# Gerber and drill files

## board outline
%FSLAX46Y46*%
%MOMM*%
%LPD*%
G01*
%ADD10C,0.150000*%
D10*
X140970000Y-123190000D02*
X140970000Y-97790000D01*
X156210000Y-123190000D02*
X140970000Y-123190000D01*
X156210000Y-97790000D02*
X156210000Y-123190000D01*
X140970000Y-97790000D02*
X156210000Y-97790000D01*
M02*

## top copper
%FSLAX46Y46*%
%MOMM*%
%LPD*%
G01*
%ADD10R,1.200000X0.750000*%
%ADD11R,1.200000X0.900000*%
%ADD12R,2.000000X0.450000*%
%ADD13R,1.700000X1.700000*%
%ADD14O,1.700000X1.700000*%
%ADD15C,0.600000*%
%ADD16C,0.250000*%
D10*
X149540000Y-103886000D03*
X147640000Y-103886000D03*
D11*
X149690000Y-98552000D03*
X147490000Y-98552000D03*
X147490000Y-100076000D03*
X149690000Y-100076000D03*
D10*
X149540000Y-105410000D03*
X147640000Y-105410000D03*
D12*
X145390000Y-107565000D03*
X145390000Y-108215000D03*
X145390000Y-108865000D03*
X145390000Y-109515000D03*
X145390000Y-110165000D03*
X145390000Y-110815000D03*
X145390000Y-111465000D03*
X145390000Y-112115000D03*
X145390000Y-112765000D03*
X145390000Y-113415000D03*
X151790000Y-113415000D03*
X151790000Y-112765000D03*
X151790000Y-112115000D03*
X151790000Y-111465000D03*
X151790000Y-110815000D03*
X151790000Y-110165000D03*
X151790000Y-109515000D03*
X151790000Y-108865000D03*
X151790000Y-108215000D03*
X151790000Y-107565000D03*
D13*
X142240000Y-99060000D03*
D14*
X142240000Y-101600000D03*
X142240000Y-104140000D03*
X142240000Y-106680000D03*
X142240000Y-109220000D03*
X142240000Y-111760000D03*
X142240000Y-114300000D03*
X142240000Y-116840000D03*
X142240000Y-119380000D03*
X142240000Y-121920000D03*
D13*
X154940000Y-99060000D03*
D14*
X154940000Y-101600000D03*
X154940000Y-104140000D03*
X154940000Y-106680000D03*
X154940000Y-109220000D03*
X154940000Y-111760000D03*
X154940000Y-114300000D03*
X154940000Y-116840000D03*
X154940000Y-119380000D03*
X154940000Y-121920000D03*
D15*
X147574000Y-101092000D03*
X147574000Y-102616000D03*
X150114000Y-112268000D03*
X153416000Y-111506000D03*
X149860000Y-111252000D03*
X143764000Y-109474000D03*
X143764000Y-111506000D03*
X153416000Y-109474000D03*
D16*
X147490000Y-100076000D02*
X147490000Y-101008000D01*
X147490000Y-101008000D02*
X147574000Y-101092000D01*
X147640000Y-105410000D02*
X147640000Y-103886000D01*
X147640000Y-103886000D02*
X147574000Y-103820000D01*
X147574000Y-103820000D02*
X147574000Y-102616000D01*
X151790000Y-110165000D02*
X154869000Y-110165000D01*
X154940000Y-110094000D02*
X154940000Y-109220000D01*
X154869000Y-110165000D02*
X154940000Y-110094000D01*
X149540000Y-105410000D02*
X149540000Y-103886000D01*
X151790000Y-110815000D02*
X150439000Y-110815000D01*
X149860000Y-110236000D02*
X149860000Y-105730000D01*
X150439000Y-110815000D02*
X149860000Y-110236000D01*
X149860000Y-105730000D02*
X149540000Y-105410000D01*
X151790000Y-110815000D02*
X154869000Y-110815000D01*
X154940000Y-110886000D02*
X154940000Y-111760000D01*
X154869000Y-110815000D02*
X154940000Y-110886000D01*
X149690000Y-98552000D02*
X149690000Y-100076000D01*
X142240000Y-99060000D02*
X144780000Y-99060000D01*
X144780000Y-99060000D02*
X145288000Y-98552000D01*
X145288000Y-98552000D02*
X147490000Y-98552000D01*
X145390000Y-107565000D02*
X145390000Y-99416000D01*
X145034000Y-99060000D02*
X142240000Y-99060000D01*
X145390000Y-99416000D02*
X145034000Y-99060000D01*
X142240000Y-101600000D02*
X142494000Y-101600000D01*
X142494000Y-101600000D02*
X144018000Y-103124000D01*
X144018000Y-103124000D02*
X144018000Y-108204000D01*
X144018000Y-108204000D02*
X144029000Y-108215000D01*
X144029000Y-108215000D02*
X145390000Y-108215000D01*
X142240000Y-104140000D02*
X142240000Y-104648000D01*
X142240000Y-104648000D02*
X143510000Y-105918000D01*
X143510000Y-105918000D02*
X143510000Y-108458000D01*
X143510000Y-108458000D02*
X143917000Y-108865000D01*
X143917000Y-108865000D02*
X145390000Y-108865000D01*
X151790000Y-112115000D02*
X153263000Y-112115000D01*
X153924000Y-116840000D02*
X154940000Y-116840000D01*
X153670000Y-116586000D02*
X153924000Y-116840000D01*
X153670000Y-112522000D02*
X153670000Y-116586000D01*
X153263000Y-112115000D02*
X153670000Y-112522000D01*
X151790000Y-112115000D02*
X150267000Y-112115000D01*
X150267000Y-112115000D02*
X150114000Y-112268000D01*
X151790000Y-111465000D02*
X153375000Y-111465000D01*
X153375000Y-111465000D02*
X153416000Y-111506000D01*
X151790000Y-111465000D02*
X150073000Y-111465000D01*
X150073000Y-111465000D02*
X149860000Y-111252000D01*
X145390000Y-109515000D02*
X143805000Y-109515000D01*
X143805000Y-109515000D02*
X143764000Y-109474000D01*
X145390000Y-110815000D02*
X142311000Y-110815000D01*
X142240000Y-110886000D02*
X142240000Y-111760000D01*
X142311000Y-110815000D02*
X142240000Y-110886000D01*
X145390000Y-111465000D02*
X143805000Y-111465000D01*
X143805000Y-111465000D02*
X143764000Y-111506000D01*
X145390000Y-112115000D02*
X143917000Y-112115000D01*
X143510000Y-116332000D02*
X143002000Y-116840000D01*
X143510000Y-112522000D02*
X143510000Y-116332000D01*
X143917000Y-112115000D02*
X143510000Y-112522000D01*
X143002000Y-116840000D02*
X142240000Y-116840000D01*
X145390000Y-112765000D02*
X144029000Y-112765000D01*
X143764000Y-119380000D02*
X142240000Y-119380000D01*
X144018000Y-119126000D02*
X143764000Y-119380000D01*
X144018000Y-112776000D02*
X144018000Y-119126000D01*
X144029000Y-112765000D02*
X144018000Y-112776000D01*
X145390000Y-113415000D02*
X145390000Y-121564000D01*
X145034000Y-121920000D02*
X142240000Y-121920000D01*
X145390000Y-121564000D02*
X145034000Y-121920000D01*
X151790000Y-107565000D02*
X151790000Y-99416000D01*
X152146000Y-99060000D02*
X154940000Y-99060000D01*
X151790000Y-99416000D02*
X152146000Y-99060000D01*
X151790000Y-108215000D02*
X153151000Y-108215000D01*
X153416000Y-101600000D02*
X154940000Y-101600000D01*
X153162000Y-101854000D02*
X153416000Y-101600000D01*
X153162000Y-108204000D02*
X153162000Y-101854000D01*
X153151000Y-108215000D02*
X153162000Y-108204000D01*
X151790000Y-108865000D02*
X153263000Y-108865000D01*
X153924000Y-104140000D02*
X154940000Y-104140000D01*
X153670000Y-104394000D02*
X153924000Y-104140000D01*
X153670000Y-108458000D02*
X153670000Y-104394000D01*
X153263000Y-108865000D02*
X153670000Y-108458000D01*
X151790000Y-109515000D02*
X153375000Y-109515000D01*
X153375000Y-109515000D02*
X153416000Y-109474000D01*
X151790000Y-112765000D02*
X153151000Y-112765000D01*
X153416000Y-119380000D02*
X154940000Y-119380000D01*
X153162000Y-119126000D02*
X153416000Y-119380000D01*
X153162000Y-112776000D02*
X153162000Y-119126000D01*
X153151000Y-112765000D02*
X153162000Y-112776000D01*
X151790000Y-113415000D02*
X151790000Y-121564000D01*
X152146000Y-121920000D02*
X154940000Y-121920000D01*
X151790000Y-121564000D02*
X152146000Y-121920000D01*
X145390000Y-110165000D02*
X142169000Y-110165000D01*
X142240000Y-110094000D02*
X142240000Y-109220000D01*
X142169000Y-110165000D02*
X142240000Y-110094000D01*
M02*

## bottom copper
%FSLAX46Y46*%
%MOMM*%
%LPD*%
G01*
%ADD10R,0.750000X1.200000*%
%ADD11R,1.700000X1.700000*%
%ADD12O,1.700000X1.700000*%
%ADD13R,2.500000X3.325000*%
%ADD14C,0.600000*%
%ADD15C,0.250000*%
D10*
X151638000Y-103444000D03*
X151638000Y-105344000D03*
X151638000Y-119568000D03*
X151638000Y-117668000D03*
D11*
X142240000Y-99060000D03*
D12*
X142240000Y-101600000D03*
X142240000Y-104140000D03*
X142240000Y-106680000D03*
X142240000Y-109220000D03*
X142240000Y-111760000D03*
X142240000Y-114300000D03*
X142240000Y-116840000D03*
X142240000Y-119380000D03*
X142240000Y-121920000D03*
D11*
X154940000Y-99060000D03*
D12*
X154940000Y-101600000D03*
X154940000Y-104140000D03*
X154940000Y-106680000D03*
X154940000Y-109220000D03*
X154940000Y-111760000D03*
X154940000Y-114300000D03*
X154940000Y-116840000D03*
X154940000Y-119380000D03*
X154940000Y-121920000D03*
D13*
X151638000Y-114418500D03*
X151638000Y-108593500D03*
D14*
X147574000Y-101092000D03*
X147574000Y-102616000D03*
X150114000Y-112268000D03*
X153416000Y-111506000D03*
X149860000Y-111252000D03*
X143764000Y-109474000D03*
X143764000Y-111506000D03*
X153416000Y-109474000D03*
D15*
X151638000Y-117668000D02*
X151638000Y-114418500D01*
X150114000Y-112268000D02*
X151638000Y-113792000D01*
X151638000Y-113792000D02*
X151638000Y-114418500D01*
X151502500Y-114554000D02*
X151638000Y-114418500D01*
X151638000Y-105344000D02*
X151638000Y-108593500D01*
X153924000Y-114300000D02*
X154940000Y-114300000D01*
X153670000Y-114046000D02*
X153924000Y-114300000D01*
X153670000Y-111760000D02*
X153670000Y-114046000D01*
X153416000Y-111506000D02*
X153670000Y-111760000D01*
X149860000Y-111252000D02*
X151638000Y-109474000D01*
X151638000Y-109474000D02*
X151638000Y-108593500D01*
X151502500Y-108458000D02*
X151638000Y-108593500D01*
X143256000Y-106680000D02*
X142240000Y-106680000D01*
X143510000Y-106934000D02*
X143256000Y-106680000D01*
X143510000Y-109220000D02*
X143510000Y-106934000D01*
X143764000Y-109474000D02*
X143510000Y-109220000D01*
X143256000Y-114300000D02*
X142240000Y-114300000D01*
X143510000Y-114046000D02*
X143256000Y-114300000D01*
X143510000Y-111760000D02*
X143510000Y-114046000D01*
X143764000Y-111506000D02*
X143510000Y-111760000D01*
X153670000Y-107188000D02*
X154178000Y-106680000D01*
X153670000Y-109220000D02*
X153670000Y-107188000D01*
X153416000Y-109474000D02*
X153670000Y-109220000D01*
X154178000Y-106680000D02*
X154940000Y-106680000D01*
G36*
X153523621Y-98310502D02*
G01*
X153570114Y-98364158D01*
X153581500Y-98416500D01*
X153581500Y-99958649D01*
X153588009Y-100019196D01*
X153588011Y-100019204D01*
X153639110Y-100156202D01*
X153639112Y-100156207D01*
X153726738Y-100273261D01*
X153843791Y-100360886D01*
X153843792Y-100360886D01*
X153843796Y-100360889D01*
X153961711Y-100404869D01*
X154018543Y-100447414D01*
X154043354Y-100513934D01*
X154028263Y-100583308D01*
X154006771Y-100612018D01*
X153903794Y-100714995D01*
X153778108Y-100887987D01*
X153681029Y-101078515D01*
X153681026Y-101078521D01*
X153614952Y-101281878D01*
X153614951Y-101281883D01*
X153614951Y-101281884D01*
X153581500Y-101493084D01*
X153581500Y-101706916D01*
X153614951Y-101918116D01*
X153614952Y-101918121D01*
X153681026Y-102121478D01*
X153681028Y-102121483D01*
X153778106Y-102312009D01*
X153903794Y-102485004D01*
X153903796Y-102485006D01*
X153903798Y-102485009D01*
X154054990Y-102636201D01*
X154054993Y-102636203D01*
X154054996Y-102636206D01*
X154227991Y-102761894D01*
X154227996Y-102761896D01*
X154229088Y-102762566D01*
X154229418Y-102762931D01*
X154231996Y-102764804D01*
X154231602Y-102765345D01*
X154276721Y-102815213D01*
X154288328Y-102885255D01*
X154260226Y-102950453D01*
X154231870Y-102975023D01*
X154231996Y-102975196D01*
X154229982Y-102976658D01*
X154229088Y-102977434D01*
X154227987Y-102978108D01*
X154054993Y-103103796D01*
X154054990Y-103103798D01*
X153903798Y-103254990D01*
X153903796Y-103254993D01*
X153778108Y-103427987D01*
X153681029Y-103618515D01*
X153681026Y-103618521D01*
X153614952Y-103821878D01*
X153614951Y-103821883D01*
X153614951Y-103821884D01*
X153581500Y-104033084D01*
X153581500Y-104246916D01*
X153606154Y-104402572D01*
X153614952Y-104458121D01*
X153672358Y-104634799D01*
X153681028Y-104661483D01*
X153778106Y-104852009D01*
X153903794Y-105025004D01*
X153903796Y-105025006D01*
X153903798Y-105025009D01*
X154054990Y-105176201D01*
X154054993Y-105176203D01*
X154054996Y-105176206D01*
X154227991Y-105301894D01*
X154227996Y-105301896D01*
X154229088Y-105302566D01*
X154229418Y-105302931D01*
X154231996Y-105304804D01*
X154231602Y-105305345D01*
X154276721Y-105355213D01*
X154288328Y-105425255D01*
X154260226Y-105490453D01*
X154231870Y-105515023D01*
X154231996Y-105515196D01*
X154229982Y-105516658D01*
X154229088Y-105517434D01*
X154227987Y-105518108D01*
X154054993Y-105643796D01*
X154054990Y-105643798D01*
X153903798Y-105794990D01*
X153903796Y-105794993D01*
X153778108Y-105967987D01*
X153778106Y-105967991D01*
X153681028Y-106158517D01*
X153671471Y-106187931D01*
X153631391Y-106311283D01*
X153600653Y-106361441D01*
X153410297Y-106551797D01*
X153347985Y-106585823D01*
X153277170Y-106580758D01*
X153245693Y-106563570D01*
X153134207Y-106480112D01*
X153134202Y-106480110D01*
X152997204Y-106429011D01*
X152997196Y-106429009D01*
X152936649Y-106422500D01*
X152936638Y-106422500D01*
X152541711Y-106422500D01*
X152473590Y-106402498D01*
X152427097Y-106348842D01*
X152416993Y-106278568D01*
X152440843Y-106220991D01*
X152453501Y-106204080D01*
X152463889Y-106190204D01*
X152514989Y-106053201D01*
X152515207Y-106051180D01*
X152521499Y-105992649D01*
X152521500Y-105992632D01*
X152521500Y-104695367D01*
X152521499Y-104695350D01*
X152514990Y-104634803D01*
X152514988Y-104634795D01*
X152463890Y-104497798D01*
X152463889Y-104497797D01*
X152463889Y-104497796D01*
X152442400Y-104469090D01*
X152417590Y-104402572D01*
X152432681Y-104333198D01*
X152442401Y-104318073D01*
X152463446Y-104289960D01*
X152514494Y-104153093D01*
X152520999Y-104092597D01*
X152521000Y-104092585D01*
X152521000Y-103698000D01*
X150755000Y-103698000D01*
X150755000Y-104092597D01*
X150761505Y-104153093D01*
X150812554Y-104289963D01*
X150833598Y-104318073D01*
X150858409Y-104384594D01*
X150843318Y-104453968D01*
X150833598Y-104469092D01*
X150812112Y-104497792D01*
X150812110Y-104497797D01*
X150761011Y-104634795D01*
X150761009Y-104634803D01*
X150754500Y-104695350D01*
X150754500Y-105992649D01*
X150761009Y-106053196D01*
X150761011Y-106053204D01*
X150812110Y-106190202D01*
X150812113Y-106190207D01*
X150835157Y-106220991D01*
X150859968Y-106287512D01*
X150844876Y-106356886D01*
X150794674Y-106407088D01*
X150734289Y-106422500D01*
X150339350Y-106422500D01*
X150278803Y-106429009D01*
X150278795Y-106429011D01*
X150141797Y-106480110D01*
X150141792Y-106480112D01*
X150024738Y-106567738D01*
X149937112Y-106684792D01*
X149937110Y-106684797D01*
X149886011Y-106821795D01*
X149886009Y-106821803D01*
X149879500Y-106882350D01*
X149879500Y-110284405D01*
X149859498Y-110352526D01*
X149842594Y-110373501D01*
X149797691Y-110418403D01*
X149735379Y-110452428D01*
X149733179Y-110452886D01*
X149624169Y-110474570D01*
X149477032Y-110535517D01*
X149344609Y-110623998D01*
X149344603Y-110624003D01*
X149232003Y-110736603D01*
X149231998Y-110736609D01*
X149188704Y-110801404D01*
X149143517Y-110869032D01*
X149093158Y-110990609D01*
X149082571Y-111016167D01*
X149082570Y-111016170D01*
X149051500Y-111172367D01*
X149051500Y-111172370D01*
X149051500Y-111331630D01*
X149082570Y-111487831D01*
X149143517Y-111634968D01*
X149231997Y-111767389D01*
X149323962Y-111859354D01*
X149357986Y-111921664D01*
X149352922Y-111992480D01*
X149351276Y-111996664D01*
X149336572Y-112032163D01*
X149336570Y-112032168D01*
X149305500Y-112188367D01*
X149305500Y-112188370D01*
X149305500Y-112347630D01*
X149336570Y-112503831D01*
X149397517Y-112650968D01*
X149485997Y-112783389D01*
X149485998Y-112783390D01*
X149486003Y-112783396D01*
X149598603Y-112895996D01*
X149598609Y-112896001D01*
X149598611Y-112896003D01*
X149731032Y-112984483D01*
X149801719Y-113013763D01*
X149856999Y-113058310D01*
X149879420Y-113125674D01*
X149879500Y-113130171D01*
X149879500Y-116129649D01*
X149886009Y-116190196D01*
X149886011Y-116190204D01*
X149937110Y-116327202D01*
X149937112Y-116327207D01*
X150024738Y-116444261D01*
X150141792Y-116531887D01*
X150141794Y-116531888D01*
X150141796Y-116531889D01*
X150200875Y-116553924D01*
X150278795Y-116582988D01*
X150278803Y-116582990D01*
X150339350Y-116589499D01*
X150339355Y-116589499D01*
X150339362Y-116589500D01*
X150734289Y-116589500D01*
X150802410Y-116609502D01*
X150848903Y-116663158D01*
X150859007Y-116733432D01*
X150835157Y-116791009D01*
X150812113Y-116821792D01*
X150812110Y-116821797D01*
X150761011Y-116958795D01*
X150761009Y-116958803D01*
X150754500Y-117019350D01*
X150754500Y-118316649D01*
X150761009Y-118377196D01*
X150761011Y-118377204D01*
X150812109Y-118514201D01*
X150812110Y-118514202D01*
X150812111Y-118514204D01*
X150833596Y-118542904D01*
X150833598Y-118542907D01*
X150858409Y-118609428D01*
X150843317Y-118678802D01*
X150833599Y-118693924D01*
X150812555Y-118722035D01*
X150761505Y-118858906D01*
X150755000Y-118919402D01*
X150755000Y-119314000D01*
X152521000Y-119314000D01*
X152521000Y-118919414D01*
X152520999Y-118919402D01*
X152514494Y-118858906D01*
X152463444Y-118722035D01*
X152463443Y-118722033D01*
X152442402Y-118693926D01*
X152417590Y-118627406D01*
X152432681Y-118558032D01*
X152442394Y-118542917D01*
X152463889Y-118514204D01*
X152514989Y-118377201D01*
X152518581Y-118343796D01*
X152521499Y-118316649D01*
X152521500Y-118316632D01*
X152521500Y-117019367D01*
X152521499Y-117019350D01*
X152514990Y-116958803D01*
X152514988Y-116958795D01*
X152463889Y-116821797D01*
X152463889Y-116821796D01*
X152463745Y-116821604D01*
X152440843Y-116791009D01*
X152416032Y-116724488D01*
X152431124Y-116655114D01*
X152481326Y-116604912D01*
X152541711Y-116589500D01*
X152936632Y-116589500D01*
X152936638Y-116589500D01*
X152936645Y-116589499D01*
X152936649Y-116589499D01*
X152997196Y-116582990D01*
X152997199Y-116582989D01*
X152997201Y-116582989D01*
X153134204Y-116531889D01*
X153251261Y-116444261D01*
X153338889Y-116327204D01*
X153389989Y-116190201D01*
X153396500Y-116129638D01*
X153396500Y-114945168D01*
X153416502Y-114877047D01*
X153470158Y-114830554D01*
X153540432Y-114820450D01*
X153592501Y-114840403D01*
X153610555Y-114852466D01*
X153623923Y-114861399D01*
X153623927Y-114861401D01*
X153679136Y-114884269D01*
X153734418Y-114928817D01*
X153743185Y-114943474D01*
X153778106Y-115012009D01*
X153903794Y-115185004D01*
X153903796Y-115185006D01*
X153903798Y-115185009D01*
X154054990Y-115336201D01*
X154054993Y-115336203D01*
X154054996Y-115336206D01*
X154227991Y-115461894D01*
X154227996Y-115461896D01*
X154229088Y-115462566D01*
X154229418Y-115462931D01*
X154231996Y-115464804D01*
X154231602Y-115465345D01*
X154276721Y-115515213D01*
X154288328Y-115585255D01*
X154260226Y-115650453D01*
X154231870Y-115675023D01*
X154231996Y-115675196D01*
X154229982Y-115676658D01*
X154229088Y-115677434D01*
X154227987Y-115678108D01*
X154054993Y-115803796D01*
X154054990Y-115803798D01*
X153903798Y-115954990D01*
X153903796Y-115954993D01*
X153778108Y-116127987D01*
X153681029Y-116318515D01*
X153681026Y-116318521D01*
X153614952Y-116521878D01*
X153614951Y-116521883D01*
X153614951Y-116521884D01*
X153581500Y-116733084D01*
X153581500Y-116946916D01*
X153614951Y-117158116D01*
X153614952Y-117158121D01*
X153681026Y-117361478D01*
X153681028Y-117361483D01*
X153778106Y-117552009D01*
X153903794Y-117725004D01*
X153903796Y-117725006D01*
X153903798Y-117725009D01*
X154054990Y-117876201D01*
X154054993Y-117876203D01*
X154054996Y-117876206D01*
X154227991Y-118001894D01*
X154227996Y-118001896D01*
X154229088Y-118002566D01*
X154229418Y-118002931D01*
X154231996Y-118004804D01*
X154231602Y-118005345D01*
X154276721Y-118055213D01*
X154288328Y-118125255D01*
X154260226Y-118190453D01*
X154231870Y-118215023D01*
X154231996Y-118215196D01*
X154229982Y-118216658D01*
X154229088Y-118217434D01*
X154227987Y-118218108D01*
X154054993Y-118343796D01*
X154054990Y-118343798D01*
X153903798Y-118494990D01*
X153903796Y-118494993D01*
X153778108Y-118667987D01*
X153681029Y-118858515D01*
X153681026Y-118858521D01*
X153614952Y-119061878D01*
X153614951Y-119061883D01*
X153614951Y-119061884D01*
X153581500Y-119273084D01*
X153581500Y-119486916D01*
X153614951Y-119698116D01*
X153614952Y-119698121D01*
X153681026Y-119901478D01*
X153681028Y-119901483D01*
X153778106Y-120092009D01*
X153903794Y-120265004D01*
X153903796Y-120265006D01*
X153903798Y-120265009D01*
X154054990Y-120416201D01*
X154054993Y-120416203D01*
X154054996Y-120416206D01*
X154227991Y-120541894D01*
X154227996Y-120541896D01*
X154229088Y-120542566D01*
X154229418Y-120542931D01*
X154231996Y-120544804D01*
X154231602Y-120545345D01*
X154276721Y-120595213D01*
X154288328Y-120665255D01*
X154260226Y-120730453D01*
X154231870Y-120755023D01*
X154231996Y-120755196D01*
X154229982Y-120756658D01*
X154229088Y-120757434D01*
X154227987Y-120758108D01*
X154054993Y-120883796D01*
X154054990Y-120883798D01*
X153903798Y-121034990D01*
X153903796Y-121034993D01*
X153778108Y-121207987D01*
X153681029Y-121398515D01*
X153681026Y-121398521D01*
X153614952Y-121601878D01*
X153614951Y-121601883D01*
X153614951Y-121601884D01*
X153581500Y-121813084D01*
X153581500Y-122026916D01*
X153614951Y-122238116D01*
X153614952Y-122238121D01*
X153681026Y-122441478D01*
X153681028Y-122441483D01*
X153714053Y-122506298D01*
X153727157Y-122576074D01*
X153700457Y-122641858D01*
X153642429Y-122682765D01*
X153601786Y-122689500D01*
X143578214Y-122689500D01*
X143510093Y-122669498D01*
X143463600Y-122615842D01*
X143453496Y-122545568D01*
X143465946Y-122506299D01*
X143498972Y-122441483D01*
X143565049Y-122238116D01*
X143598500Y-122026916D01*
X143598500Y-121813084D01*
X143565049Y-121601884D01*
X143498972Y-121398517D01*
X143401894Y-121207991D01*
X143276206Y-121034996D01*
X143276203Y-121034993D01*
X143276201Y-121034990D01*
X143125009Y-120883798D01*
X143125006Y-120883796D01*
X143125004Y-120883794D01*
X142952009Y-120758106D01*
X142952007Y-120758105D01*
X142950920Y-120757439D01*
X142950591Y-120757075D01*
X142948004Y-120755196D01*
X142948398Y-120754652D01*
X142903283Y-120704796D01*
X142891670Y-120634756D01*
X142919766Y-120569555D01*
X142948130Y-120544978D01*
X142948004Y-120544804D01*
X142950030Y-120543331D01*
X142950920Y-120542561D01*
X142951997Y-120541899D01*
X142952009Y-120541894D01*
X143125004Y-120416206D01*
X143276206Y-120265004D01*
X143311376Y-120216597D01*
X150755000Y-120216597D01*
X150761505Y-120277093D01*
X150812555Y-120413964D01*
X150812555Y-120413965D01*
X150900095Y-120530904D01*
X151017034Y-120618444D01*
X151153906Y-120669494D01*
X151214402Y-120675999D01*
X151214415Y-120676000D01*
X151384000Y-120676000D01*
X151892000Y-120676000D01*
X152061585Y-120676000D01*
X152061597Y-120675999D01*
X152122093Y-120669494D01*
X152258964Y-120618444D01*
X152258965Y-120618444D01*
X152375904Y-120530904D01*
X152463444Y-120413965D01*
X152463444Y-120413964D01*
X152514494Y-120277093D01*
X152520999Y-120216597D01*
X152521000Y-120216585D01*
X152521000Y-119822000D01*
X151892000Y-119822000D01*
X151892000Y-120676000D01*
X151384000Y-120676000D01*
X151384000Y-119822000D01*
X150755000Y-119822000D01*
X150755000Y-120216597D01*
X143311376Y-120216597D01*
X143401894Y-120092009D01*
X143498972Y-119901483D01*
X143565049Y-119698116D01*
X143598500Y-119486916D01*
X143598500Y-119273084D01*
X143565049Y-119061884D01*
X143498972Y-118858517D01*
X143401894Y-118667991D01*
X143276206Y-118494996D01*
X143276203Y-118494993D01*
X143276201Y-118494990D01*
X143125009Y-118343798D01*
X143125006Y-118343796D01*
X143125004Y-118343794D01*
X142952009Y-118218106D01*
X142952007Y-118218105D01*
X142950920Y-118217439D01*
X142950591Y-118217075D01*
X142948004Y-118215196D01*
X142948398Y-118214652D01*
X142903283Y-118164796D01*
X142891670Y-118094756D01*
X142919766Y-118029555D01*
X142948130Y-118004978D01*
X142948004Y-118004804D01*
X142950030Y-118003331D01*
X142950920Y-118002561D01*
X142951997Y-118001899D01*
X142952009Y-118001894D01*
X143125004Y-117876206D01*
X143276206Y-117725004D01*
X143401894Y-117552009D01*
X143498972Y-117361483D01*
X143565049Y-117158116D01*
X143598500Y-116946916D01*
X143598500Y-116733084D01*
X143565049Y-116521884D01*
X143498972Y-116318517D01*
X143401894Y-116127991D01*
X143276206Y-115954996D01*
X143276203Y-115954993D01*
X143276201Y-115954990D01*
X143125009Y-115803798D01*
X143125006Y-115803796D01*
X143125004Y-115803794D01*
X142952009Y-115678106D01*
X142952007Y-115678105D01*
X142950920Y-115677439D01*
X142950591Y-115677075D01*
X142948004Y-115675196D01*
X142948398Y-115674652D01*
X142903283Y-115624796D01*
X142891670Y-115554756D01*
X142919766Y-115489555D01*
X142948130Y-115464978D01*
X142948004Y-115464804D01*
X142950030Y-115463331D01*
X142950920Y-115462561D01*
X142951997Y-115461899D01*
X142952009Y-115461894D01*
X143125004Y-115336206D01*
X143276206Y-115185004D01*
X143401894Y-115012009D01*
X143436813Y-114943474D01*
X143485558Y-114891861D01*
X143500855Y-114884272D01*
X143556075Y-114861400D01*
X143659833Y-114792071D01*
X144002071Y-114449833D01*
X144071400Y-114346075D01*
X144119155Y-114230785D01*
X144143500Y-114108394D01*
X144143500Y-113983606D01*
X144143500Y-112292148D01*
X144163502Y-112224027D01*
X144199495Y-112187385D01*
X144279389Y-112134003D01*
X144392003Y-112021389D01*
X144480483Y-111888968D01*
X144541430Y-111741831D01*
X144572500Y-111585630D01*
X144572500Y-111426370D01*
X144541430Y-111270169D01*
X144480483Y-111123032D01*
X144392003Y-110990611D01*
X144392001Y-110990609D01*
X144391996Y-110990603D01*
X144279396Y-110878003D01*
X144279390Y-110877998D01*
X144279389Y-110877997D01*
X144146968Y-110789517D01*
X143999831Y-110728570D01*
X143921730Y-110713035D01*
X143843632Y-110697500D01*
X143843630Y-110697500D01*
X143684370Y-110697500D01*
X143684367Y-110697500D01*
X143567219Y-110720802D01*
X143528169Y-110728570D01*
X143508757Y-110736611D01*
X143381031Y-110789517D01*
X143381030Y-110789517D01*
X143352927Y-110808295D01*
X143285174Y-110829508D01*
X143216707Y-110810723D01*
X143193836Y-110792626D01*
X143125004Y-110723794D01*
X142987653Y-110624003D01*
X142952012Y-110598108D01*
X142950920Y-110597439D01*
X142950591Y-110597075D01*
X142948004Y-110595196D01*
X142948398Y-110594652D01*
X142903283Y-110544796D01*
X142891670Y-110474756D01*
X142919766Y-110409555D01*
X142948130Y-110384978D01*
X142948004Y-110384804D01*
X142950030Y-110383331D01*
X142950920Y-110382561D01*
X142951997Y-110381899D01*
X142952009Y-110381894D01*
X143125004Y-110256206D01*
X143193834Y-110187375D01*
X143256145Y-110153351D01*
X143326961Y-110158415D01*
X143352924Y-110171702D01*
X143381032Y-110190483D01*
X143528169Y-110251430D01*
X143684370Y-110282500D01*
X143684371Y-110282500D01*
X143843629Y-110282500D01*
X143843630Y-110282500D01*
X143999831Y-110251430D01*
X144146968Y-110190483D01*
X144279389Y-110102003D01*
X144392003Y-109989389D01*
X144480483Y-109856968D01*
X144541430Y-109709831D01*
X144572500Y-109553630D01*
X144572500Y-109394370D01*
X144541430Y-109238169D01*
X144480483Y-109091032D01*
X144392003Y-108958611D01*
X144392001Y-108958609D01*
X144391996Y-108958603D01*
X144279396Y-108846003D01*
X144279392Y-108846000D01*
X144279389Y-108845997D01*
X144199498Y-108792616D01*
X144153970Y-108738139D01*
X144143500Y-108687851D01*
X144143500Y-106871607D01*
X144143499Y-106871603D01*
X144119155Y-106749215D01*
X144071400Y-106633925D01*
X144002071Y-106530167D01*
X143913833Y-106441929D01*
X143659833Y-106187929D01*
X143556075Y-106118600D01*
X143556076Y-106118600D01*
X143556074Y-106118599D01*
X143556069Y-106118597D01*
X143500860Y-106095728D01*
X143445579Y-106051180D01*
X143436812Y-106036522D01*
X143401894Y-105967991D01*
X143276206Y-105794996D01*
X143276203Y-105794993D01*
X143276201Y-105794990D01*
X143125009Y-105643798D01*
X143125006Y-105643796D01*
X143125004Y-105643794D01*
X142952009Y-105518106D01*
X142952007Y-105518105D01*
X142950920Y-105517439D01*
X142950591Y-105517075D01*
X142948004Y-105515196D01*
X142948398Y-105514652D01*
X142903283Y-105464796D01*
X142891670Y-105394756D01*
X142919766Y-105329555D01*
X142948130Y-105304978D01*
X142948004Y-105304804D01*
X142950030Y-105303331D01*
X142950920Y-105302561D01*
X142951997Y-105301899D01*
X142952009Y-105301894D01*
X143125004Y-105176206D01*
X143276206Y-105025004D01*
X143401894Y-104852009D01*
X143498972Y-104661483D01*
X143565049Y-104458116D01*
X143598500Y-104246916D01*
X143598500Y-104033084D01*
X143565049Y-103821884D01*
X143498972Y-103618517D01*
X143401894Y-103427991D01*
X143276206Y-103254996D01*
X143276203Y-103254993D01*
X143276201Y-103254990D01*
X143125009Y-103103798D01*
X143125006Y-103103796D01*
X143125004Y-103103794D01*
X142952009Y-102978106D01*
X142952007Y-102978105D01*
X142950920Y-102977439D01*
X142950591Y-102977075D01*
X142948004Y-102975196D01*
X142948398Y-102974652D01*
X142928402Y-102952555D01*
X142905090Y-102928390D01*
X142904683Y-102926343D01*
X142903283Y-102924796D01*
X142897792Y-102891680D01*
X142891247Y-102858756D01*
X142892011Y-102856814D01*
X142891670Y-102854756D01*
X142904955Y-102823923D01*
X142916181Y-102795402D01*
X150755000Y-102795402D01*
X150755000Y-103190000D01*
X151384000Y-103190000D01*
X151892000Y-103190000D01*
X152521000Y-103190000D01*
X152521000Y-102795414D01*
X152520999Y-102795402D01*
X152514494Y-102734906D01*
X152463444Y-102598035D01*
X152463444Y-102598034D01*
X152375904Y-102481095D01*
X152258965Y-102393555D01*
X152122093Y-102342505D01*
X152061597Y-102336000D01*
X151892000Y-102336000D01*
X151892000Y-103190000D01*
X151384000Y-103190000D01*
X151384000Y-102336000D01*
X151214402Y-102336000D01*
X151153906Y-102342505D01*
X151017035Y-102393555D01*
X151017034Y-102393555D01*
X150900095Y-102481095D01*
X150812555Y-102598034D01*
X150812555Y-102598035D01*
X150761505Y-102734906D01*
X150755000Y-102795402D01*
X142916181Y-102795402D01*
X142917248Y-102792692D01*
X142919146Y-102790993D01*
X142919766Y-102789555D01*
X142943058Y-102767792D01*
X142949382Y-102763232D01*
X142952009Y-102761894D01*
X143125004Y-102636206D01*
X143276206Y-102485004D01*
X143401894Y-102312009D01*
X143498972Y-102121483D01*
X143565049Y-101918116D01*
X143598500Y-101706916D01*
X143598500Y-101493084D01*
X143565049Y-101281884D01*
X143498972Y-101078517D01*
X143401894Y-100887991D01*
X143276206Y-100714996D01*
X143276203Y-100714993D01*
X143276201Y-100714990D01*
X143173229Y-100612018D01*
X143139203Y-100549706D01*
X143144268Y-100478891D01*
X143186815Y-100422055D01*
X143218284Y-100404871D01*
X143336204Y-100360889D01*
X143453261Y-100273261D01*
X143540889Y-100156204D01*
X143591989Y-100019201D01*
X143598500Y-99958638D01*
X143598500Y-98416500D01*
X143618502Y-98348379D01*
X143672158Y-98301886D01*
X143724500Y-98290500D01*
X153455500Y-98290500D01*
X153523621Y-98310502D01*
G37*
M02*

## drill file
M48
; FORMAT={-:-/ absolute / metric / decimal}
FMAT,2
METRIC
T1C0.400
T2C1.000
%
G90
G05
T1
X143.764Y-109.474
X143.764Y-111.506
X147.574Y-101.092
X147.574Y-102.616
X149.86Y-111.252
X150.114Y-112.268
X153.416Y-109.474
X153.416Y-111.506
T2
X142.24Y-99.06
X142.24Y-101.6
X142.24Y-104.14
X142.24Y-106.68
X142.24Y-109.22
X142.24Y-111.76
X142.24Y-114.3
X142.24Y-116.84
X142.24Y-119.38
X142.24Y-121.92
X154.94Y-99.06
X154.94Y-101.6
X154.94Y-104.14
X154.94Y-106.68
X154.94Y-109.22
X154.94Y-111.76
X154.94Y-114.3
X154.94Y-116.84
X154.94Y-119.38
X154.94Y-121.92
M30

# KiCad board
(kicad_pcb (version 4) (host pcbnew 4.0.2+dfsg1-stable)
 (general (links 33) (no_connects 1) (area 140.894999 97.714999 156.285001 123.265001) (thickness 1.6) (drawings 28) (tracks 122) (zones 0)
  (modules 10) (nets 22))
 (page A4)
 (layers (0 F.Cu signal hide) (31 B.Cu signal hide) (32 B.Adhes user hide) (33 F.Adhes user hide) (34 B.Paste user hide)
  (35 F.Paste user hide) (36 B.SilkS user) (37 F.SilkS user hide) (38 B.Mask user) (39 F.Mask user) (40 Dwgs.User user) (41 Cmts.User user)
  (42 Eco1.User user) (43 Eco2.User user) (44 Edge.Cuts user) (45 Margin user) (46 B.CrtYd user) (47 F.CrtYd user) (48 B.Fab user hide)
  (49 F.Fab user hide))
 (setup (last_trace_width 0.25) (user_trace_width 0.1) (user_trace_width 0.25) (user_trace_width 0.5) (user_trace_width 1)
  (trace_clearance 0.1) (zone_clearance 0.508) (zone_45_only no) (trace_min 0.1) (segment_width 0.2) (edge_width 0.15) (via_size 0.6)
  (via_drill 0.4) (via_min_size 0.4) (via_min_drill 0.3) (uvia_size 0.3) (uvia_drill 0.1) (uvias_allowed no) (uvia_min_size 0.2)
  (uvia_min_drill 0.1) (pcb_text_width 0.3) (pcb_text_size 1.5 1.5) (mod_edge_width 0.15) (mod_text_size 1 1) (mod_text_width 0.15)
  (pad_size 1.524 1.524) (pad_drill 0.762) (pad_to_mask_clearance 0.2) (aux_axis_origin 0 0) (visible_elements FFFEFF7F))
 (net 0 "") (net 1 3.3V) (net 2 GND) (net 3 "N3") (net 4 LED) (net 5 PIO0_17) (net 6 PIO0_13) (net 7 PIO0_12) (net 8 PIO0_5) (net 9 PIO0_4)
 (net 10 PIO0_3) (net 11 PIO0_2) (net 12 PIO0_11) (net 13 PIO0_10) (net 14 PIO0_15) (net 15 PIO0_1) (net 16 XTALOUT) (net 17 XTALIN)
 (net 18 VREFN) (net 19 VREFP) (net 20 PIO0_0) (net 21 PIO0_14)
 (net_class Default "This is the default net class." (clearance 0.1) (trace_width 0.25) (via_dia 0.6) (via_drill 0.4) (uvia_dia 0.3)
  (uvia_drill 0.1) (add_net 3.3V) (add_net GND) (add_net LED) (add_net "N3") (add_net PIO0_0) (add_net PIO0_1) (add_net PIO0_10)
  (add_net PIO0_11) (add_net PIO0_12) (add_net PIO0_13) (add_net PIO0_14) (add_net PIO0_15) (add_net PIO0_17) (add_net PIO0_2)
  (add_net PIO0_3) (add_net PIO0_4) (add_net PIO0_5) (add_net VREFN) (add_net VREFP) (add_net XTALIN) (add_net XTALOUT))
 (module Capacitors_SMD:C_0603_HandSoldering (layer F.Cu) (at 148.59 103.886 180)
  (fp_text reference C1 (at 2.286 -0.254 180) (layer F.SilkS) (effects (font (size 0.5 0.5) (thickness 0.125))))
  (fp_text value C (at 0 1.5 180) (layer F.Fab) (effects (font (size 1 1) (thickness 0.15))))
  (pad 1 smd rect (at -0.95 0 180) (size 1.2 0.75) (layers F.Cu F.Paste F.Mask) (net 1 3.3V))
  (pad 2 smd rect (at 0.95 0 180) (size 1.2 0.75) (layers F.Cu F.Paste F.Mask) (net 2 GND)))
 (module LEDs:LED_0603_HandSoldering (layer F.Cu) (at 148.59 98.552 180)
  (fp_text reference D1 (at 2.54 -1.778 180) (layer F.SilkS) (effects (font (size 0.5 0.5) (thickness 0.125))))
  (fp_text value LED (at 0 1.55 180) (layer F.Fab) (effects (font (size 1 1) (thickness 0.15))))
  (pad 1 smd rect (at -1.1 0 180) (size 1.2 0.9) (layers F.Cu F.Paste F.Mask) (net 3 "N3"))
  (pad 2 smd rect (at 1.1 0 180) (size 1.2 0.9) (layers F.Cu F.Paste F.Mask) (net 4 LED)))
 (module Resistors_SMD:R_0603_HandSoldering (layer F.Cu) (at 148.59 100.076)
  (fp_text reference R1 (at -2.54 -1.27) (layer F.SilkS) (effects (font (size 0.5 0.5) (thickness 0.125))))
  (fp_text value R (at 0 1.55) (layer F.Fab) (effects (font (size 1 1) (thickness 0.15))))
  (pad 1 smd rect (at -1.1 0) (size 1.2 0.9) (layers F.Cu F.Paste F.Mask) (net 2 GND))
  (pad 2 smd rect (at 1.1 0) (size 1.2 0.9) (layers F.Cu F.Paste F.Mask) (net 3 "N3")))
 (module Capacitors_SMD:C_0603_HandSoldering (layer F.Cu) (at 148.59 105.41 180)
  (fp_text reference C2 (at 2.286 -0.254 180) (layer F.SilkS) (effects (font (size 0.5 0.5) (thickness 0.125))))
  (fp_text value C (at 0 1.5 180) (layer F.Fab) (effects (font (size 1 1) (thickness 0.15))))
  (pad 1 smd rect (at -0.95 0 180) (size 1.2 0.75) (layers F.Cu F.Paste F.Mask) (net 1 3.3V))
  (pad 2 smd rect (at 0.95 0 180) (size 1.2 0.75) (layers F.Cu F.Paste F.Mask) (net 2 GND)))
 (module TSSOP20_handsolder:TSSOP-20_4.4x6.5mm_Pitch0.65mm (layer F.Cu) (at 148.59 110.49)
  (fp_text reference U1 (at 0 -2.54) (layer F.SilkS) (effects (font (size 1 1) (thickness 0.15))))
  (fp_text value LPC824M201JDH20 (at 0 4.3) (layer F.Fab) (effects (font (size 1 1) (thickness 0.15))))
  (pad 1 smd rect (at -3.2 -2.925) (size 2 0.45) (layers F.Cu F.Paste F.Mask) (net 4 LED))
  (pad 2 smd rect (at -3.2 -2.275) (size 2 0.45) (layers F.Cu F.Paste F.Mask) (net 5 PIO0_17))
  (pad 3 smd rect (at -3.2 -1.625) (size 2 0.45) (layers F.Cu F.Paste F.Mask) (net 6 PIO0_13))
  (pad 4 smd rect (at -3.2 -0.975) (size 2 0.45) (layers F.Cu F.Paste F.Mask) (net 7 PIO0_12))
  (pad 5 smd rect (at -3.2 -0.325) (size 2 0.45) (layers F.Cu F.Paste F.Mask) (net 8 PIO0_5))
  (pad 6 smd rect (at -3.2 0.325) (size 2 0.45) (layers F.Cu F.Paste F.Mask) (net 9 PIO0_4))
  (pad 7 smd rect (at -3.2 0.975) (size 2 0.45) (layers F.Cu F.Paste F.Mask) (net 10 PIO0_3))
  (pad 8 smd rect (at -3.2 1.625) (size 2 0.45) (layers F.Cu F.Paste F.Mask) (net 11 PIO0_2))
  (pad 9 smd rect (at -3.2 2.275) (size 2 0.45) (layers F.Cu F.Paste F.Mask) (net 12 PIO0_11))
  (pad 10 smd rect (at -3.2 2.925) (size 2 0.45) (layers F.Cu F.Paste F.Mask) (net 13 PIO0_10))
  (pad 11 smd rect (at 3.2 2.925) (size 2 0.45) (layers F.Cu F.Paste F.Mask) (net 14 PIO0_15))
  (pad 12 smd rect (at 3.2 2.275) (size 2 0.45) (layers F.Cu F.Paste F.Mask) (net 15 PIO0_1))
  (pad 13 smd rect (at 3.2 1.625) (size 2 0.45) (layers F.Cu F.Paste F.Mask) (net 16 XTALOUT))
  (pad 14 smd rect (at 3.2 0.975) (size 2 0.45) (layers F.Cu F.Paste F.Mask) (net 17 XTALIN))
  (pad 15 smd rect (at 3.2 0.325) (size 2 0.45) (layers F.Cu F.Paste F.Mask) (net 1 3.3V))
  (pad 16 smd rect (at 3.2 -0.325) (size 2 0.45) (layers F.Cu F.Paste F.Mask) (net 2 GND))
  (pad 17 smd rect (at 3.2 -0.975) (size 2 0.45) (layers F.Cu F.Paste F.Mask) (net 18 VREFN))
  (pad 18 smd rect (at 3.2 -1.625) (size 2 0.45) (layers F.Cu F.Paste F.Mask) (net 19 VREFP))
  (pad 19 smd rect (at 3.2 -2.275) (size 2 0.45) (layers F.Cu F.Paste F.Mask) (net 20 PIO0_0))
  (pad 20 smd rect (at 3.2 -2.925) (size 2 0.45) (layers F.Cu F.Paste F.Mask) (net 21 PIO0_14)))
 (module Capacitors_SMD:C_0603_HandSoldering (layer B.Cu) (at 151.638 104.394 270)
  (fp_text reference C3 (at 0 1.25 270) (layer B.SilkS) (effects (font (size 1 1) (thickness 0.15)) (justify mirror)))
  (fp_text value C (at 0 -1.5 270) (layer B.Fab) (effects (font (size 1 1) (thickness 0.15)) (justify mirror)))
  (pad 1 smd rect (at -0.95 0 270) (size 1.2 0.75) (layers B.Cu B.Paste B.Mask) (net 2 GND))
  (pad 2 smd rect (at 0.95 0 270) (size 1.2 0.75) (layers B.Cu B.Paste B.Mask) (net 17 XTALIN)))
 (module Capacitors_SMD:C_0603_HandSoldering (layer B.Cu) (at 151.638 118.618 90)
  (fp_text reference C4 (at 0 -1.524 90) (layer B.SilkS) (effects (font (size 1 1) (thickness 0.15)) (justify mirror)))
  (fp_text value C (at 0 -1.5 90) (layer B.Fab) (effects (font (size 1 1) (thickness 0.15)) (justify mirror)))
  (pad 1 smd rect (at -0.95 0 90) (size 1.2 0.75) (layers B.Cu B.Paste B.Mask) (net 2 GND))
  (pad 2 smd rect (at 0.95 0 90) (size 1.2 0.75) (layers B.Cu B.Paste B.Mask) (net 16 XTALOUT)))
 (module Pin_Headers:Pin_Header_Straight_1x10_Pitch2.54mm (layer F.Cu) (at 142.24 99.06)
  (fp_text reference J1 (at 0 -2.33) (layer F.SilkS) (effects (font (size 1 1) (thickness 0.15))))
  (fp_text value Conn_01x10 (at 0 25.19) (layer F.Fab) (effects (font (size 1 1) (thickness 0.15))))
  (pad 1 thru_hole rect (at 0 0) (size 1.7 1.7) (drill 1) (layers *.Cu *.Mask) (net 4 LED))
  (pad 2 thru_hole oval (at 0 2.54) (size 1.7 1.7) (drill 1) (layers *.Cu *.Mask) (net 5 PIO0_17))
  (pad 3 thru_hole oval (at 0 5.08) (size 1.7 1.7) (drill 1) (layers *.Cu *.Mask) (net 6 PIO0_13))
  (pad 4 thru_hole oval (at 0 7.62) (size 1.7 1.7) (drill 1) (layers *.Cu *.Mask) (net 7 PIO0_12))
  (pad 5 thru_hole oval (at 0 10.16) (size 1.7 1.7) (drill 1) (layers *.Cu *.Mask) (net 8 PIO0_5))
  (pad 6 thru_hole oval (at 0 12.7) (size 1.7 1.7) (drill 1) (layers *.Cu *.Mask) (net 9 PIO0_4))
  (pad 7 thru_hole oval (at 0 15.24) (size 1.7 1.7) (drill 1) (layers *.Cu *.Mask) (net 10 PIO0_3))
  (pad 8 thru_hole oval (at 0 17.78) (size 1.7 1.7) (drill 1) (layers *.Cu *.Mask) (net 11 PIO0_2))
  (pad 9 thru_hole oval (at 0 20.32) (size 1.7 1.7) (drill 1) (layers *.Cu *.Mask) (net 12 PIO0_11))
  (pad 10 thru_hole oval (at 0 22.86) (size 1.7 1.7) (drill 1) (layers *.Cu *.Mask) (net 13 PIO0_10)))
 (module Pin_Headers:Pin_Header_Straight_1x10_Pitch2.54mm (layer F.Cu) (at 154.94 99.06)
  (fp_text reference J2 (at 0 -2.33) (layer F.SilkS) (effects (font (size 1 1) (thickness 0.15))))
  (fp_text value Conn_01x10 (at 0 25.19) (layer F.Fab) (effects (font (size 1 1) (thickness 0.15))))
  (pad 1 thru_hole rect (at 0 0) (size 1.7 1.7) (drill 1) (layers *.Cu *.Mask) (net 21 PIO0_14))
  (pad 2 thru_hole oval (at 0 2.54) (size 1.7 1.7) (drill 1) (layers *.Cu *.Mask) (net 20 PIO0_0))
  (pad 3 thru_hole oval (at 0 5.08) (size 1.7 1.7) (drill 1) (layers *.Cu *.Mask) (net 19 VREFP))
  (pad 4 thru_hole oval (at 0 7.62) (size 1.7 1.7) (drill 1) (layers *.Cu *.Mask) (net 18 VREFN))
  (pad 5 thru_hole oval (at 0 10.16) (size 1.7 1.7) (drill 1) (layers *.Cu *.Mask) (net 2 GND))
  (pad 6 thru_hole oval (at 0 12.7) (size 1.7 1.7) (drill 1) (layers *.Cu *.Mask) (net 1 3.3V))
  (pad 7 thru_hole oval (at 0 15.24) (size 1.7 1.7) (drill 1) (layers *.Cu *.Mask) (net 17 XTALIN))
  (pad 8 thru_hole oval (at 0 17.78) (size 1.7 1.7) (drill 1) (layers *.Cu *.Mask) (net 16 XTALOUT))
  (pad 9 thru_hole oval (at 0 20.32) (size 1.7 1.7) (drill 1) (layers *.Cu *.Mask) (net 15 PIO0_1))
  (pad 10 thru_hole oval (at 0 22.86) (size 1.7 1.7) (drill 1) (layers *.Cu *.Mask) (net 14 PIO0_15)))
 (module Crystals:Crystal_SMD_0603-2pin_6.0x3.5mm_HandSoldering (layer B.Cu) (at 151.638 111.506 90)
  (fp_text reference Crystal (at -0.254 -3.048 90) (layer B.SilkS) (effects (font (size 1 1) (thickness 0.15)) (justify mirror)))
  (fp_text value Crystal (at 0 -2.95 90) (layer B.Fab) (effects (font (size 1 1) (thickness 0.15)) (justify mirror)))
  (pad 1 smd rect (at -2.9125 0 90) (size 3.325 2.5) (layers B.Cu B.Paste B.Mask) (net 16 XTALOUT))
  (pad 2 smd rect (at 2.9125 0 90) (size 3.325 2.5) (layers B.Cu B.Paste B.Mask) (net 17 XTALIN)))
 (gr_line (start 140.97 123.19) (end 140.97 97.79) (angle 90) (layer Edge.Cuts) (width 0.15))
 (gr_line (start 156.21 123.19) (end 140.97 123.19) (angle 90) (layer Edge.Cuts) (width 0.15))
 (gr_line (start 156.21 97.79) (end 156.21 123.19) (angle 90) (layer Edge.Cuts) (width 0.15))
 (gr_line (start 140.97 97.79) (end 156.21 97.79) (angle 90) (layer Edge.Cuts) (width 0.15))
 (segment (start 147.49 100.076) (end 147.49 101.008) (width 0.25) (layer F.Cu) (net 2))
 (via (at 147.574 101.092) (size 0.6) (drill 0.4) (layers F.Cu B.Cu) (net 2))
 (segment (start 147.49 101.008) (end 147.574 101.092) (width 0.25) (layer F.Cu) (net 2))
 (segment (start 147.64 105.41) (end 147.64 103.886) (width 0.25) (layer F.Cu) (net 2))
 (segment (start 147.64 103.886) (end 147.574 103.82) (width 0.25) (layer F.Cu) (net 2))
 (segment (start 147.574 103.82) (end 147.574 102.616) (width 0.25) (layer F.Cu) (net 2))
 (via (at 147.574 102.616) (size 0.6) (drill 0.4) (layers F.Cu B.Cu) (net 2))
 (segment (start 151.79 110.165) (end 154.869 110.165) (width 0.25) (layer F.Cu) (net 2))
 (segment (start 154.94 110.094) (end 154.94 109.22) (width 0.25) (layer F.Cu) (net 2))
 (segment (start 154.869 110.165) (end 154.94 110.094) (width 0.25) (layer F.Cu) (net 2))
 (segment (start 149.54 105.41) (end 149.54 103.886) (width 0.25) (layer F.Cu) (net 1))
 (segment (start 151.79 110.815) (end 150.439 110.815) (width 0.25) (layer F.Cu) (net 1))
 (segment (start 149.86 110.236) (end 149.86 105.73) (width 0.25) (layer F.Cu) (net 1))
 (segment (start 150.439 110.815) (end 149.86 110.236) (width 0.25) (layer F.Cu) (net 1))
 (segment (start 149.86 105.73) (end 149.54 105.41) (width 0.25) (layer F.Cu) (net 1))
 (segment (start 151.79 110.815) (end 154.869 110.815) (width 0.25) (layer F.Cu) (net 1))
 (segment (start 154.94 110.886) (end 154.94 111.76) (width 0.25) (layer F.Cu) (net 1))
 (segment (start 154.869 110.815) (end 154.94 110.886) (width 0.25) (layer F.Cu) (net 1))
 (segment (start 149.69 98.552) (end 149.69 100.076) (width 0.25) (layer F.Cu) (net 3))
 (segment (start 142.24 99.06) (end 144.78 99.06) (width 0.25) (layer F.Cu) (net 4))
 (segment (start 144.78 99.06) (end 145.288 98.552) (width 0.25) (layer F.Cu) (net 4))
 (segment (start 145.288 98.552) (end 147.49 98.552) (width 0.25) (layer F.Cu) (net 4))
 (segment (start 145.39 107.565) (end 145.39 99.416) (width 0.25) (layer F.Cu) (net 4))
 (segment (start 145.034 99.06) (end 142.24 99.06) (width 0.25) (layer F.Cu) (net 4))
 (segment (start 145.39 99.416) (end 145.034 99.06) (width 0.25) (layer F.Cu) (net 4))
 (segment (start 142.24 101.6) (end 142.494 101.6) (width 0.25) (layer F.Cu) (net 5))
 (segment (start 142.494 101.6) (end 144.018 103.124) (width 0.25) (layer F.Cu) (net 5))
 (segment (start 144.018 103.124) (end 144.018 108.204) (width 0.25) (layer F.Cu) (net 5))
 (segment (start 144.018 108.204) (end 144.029 108.215) (width 0.25) (layer F.Cu) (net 5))
 (segment (start 144.029 108.215) (end 145.39 108.215) (width 0.25) (layer F.Cu) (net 5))
 (segment (start 142.24 104.14) (end 142.24 104.648) (width 0.25) (layer F.Cu) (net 6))
 (segment (start 142.24 104.648) (end 143.51 105.918) (width 0.25) (layer F.Cu) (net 6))
 (segment (start 143.51 105.918) (end 143.51 108.458) (width 0.25) (layer F.Cu) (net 6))
 (segment (start 143.51 108.458) (end 143.917 108.865) (width 0.25) (layer F.Cu) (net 6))
 (segment (start 143.917 108.865) (end 145.39 108.865) (width 0.25) (layer F.Cu) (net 6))
 (segment (start 151.638 117.668) (end 151.638 114.4185) (width 0.25) (layer B.Cu) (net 16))
 (segment (start 151.79 112.115) (end 153.263 112.115) (width 0.25) (layer F.Cu) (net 16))
 (segment (start 153.924 116.84) (end 154.94 116.84) (width 0.25) (layer F.Cu) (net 16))
 (segment (start 153.67 116.586) (end 153.924 116.84) (width 0.25) (layer F.Cu) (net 16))
 (segment (start 153.67 112.522) (end 153.67 116.586) (width 0.25) (layer F.Cu) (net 16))
 (segment (start 153.263 112.115) (end 153.67 112.522) (width 0.25) (layer F.Cu) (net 16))
 (segment (start 151.79 112.115) (end 150.267 112.115) (width 0.25) (layer F.Cu) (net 16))
 (segment (start 150.114 112.268) (end 151.638 113.792) (width 0.25) (layer B.Cu) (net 16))
 (via (at 150.114 112.268) (size 0.6) (drill 0.4) (layers F.Cu B.Cu) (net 16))
 (segment (start 150.267 112.115) (end 150.114 112.268) (width 0.25) (layer F.Cu) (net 16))
 (segment (start 151.638 113.792) (end 151.638 114.4185) (width 0.25) (layer B.Cu) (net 16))
 (segment (start 151.5025 114.554) (end 151.638 114.4185) (width 0.25) (layer B.Cu) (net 16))
 (segment (start 151.638 105.344) (end 151.638 108.5935) (width 0.25) (layer B.Cu) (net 17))
 (segment (start 151.79 111.465) (end 153.375 111.465) (width 0.25) (layer F.Cu) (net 17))
 (segment (start 153.924 114.3) (end 154.94 114.3) (width 0.25) (layer B.Cu) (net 17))
 (segment (start 153.67 114.046) (end 153.924 114.3) (width 0.25) (layer B.Cu) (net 17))
 (segment (start 153.67 111.76) (end 153.67 114.046) (width 0.25) (layer B.Cu) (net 17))
 (segment (start 153.416 111.506) (end 153.67 111.76) (width 0.25) (layer B.Cu) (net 17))
 (via (at 153.416 111.506) (size 0.6) (drill 0.4) (layers F.Cu B.Cu) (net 17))
 (segment (start 153.375 111.465) (end 153.416 111.506) (width 0.25) (layer F.Cu) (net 17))
 (segment (start 151.79 111.465) (end 150.073 111.465) (width 0.25) (layer F.Cu) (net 17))
 (segment (start 149.86 111.252) (end 151.638 109.474) (width 0.25) (layer B.Cu) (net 17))
 (via (at 149.86 111.252) (size 0.6) (drill 0.4) (layers F.Cu B.Cu) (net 17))
 (segment (start 150.073 111.465) (end 149.86 111.252) (width 0.25) (layer F.Cu) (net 17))
 (segment (start 151.638 109.474) (end 151.638 108.5935) (width 0.25) (layer B.Cu) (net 17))
 (segment (start 151.5025 108.458) (end 151.638 108.5935) (width 0.25) (layer B.Cu) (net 17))
 (segment (start 145.39 109.515) (end 143.805 109.515) (width 0.25) (layer F.Cu) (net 7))
 (segment (start 143.256 106.68) (end 142.24 106.68) (width 0.25) (layer B.Cu) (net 7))
 (segment (start 143.51 106.934) (end 143.256 106.68) (width 0.25) (layer B.Cu) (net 7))
 (segment (start 143.51 109.22) (end 143.51 106.934) (width 0.25) (layer B.Cu) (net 7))
 (segment (start 143.764 109.474) (end 143.51 109.22) (width 0.25) (layer B.Cu) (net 7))
 (via (at 143.764 109.474) (size 0.6) (drill 0.4) (layers F.Cu B.Cu) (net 7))
 (segment (start 143.805 109.515) (end 143.764 109.474) (width 0.25) (layer F.Cu) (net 7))
 (segment (start 145.39 110.815) (end 142.311 110.815) (width 0.25) (layer F.Cu) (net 9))
 (segment (start 142.24 110.886) (end 142.24 111.76) (width 0.25) (layer F.Cu) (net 9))
 (segment (start 142.311 110.815) (end 142.24 110.886) (width 0.25) (layer F.Cu) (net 9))
 (segment (start 145.39 111.465) (end 143.805 111.465) (width 0.25) (layer F.Cu) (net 10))
 (segment (start 143.256 114.3) (end 142.24 114.3) (width 0.25) (layer B.Cu) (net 10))
 (segment (start 143.51 114.046) (end 143.256 114.3) (width 0.25) (layer B.Cu) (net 10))
 (segment (start 143.51 111.76) (end 143.51 114.046) (width 0.25) (layer B.Cu) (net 10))
 (segment (start 143.764 111.506) (end 143.51 111.76) (width 0.25) (layer B.Cu) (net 10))
 (via (at 143.764 111.506) (size 0.6) (drill 0.4) (layers F.Cu B.Cu) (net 10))
 (segment (start 143.805 111.465) (end 143.764 111.506) (width 0.25) (layer F.Cu) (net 10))
 (segment (start 145.39 112.115) (end 143.917 112.115) (width 0.25) (layer F.Cu) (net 11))
 (segment (start 143.51 116.332) (end 143.002 116.84) (width 0.25) (layer F.Cu) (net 11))
 (segment (start 143.51 112.522) (end 143.51 116.332) (width 0.25) (layer F.Cu) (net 11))
 (segment (start 143.917 112.115) (end 143.51 112.522) (width 0.25) (layer F.Cu) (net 11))
 (segment (start 143.002 116.84) (end 142.24 116.84) (width 0.25) (layer F.Cu) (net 11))
 (segment (start 145.39 112.765) (end 144.029 112.765) (width 0.25) (layer F.Cu) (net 12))
 (segment (start 143.764 119.38) (end 142.24 119.38) (width 0.25) (layer F.Cu) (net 12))
 (segment (start 144.018 119.126) (end 143.764 119.38) (width 0.25) (layer F.Cu) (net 12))
 (segment (start 144.018 112.776) (end 144.018 119.126) (width 0.25) (layer F.Cu) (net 12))
 (segment (start 144.029 112.765) (end 144.018 112.776) (width 0.25) (layer F.Cu) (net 12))
 (segment (start 145.39 113.415) (end 145.39 121.564) (width 0.25) (layer F.Cu) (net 13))
 (segment (start 145.034 121.92) (end 142.24 121.92) (width 0.25) (layer F.Cu) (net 13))
 (segment (start 145.39 121.564) (end 145.034 121.92) (width 0.25) (layer F.Cu) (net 13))
 (segment (start 151.79 107.565) (end 151.79 99.416) (width 0.25) (layer F.Cu) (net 21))
 (segment (start 152.146 99.06) (end 154.94 99.06) (width 0.25) (layer F.Cu) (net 21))
 (segment (start 151.79 99.416) (end 152.146 99.06) (width 0.25) (layer F.Cu) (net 21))
 (segment (start 151.79 108.215) (end 153.151 108.215) (width 0.25) (layer F.Cu) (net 20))
 (segment (start 153.416 101.6) (end 154.94 101.6) (width 0.25) (layer F.Cu) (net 20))
 (segment (start 153.162 101.854) (end 153.416 101.6) (width 0.25) (layer F.Cu) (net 20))
 (segment (start 153.162 108.204) (end 153.162 101.854) (width 0.25) (layer F.Cu) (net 20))
 (segment (start 153.151 108.215) (end 153.162 108.204) (width 0.25) (layer F.Cu) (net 20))
 (segment (start 151.79 108.865) (end 153.263 108.865) (width 0.25) (layer F.Cu) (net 19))
 (segment (start 153.924 104.14) (end 154.94 104.14) (width 0.25) (layer F.Cu) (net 19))
 (segment (start 153.67 104.394) (end 153.924 104.14) (width 0.25) (layer F.Cu) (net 19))
 (segment (start 153.67 108.458) (end 153.67 104.394) (width 0.25) (layer F.Cu) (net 19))
 (segment (start 153.263 108.865) (end 153.67 108.458) (width 0.25) (layer F.Cu) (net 19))
 (segment (start 151.79 109.515) (end 153.375 109.515) (width 0.25) (layer F.Cu) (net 18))
 (segment (start 153.67 107.188) (end 154.178 106.68) (width 0.25) (layer B.Cu) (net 18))
 (segment (start 153.67 109.22) (end 153.67 107.188) (width 0.25) (layer B.Cu) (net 18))
 (segment (start 153.416 109.474) (end 153.67 109.22) (width 0.25) (layer B.Cu) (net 18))
 (via (at 153.416 109.474) (size 0.6) (drill 0.4) (layers F.Cu B.Cu) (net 18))
 (segment (start 153.375 109.515) (end 153.416 109.474) (width 0.25) (layer F.Cu) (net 18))
 (segment (start 154.178 106.68) (end 154.94 106.68) (width 0.25) (layer B.Cu) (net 18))
 (segment (start 151.79 112.765) (end 153.151 112.765) (width 0.25) (layer F.Cu) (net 15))
 (segment (start 153.416 119.38) (end 154.94 119.38) (width 0.25) (layer F.Cu) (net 15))
 (segment (start 153.162 119.126) (end 153.416 119.38) (width 0.25) (layer F.Cu) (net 15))
 (segment (start 153.162 112.776) (end 153.162 119.126) (width 0.25) (layer F.Cu) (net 15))
 (segment (start 153.151 112.765) (end 153.162 112.776) (width 0.25) (layer F.Cu) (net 15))
 (segment (start 151.79 113.415) (end 151.79 121.564) (width 0.25) (layer F.Cu) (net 14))
 (segment (start 152.146 121.92) (end 154.94 121.92) (width 0.25) (layer F.Cu) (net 14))
 (segment (start 151.79 121.564) (end 152.146 121.92) (width 0.25) (layer F.Cu) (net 14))
 (segment (start 145.39 110.165) (end 142.169 110.165) (width 0.25) (layer F.Cu) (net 8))
 (segment (start 142.24 110.094) (end 142.24 109.22) (width 0.25) (layer F.Cu) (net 8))
 (segment (start 142.169 110.165) (end 142.24 110.094) (width 0.25) (layer F.Cu) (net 8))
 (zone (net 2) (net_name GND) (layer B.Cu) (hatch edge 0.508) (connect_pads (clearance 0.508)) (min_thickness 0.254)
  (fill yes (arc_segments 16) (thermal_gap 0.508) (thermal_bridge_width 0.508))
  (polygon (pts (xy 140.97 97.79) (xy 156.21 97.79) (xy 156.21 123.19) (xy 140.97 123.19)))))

